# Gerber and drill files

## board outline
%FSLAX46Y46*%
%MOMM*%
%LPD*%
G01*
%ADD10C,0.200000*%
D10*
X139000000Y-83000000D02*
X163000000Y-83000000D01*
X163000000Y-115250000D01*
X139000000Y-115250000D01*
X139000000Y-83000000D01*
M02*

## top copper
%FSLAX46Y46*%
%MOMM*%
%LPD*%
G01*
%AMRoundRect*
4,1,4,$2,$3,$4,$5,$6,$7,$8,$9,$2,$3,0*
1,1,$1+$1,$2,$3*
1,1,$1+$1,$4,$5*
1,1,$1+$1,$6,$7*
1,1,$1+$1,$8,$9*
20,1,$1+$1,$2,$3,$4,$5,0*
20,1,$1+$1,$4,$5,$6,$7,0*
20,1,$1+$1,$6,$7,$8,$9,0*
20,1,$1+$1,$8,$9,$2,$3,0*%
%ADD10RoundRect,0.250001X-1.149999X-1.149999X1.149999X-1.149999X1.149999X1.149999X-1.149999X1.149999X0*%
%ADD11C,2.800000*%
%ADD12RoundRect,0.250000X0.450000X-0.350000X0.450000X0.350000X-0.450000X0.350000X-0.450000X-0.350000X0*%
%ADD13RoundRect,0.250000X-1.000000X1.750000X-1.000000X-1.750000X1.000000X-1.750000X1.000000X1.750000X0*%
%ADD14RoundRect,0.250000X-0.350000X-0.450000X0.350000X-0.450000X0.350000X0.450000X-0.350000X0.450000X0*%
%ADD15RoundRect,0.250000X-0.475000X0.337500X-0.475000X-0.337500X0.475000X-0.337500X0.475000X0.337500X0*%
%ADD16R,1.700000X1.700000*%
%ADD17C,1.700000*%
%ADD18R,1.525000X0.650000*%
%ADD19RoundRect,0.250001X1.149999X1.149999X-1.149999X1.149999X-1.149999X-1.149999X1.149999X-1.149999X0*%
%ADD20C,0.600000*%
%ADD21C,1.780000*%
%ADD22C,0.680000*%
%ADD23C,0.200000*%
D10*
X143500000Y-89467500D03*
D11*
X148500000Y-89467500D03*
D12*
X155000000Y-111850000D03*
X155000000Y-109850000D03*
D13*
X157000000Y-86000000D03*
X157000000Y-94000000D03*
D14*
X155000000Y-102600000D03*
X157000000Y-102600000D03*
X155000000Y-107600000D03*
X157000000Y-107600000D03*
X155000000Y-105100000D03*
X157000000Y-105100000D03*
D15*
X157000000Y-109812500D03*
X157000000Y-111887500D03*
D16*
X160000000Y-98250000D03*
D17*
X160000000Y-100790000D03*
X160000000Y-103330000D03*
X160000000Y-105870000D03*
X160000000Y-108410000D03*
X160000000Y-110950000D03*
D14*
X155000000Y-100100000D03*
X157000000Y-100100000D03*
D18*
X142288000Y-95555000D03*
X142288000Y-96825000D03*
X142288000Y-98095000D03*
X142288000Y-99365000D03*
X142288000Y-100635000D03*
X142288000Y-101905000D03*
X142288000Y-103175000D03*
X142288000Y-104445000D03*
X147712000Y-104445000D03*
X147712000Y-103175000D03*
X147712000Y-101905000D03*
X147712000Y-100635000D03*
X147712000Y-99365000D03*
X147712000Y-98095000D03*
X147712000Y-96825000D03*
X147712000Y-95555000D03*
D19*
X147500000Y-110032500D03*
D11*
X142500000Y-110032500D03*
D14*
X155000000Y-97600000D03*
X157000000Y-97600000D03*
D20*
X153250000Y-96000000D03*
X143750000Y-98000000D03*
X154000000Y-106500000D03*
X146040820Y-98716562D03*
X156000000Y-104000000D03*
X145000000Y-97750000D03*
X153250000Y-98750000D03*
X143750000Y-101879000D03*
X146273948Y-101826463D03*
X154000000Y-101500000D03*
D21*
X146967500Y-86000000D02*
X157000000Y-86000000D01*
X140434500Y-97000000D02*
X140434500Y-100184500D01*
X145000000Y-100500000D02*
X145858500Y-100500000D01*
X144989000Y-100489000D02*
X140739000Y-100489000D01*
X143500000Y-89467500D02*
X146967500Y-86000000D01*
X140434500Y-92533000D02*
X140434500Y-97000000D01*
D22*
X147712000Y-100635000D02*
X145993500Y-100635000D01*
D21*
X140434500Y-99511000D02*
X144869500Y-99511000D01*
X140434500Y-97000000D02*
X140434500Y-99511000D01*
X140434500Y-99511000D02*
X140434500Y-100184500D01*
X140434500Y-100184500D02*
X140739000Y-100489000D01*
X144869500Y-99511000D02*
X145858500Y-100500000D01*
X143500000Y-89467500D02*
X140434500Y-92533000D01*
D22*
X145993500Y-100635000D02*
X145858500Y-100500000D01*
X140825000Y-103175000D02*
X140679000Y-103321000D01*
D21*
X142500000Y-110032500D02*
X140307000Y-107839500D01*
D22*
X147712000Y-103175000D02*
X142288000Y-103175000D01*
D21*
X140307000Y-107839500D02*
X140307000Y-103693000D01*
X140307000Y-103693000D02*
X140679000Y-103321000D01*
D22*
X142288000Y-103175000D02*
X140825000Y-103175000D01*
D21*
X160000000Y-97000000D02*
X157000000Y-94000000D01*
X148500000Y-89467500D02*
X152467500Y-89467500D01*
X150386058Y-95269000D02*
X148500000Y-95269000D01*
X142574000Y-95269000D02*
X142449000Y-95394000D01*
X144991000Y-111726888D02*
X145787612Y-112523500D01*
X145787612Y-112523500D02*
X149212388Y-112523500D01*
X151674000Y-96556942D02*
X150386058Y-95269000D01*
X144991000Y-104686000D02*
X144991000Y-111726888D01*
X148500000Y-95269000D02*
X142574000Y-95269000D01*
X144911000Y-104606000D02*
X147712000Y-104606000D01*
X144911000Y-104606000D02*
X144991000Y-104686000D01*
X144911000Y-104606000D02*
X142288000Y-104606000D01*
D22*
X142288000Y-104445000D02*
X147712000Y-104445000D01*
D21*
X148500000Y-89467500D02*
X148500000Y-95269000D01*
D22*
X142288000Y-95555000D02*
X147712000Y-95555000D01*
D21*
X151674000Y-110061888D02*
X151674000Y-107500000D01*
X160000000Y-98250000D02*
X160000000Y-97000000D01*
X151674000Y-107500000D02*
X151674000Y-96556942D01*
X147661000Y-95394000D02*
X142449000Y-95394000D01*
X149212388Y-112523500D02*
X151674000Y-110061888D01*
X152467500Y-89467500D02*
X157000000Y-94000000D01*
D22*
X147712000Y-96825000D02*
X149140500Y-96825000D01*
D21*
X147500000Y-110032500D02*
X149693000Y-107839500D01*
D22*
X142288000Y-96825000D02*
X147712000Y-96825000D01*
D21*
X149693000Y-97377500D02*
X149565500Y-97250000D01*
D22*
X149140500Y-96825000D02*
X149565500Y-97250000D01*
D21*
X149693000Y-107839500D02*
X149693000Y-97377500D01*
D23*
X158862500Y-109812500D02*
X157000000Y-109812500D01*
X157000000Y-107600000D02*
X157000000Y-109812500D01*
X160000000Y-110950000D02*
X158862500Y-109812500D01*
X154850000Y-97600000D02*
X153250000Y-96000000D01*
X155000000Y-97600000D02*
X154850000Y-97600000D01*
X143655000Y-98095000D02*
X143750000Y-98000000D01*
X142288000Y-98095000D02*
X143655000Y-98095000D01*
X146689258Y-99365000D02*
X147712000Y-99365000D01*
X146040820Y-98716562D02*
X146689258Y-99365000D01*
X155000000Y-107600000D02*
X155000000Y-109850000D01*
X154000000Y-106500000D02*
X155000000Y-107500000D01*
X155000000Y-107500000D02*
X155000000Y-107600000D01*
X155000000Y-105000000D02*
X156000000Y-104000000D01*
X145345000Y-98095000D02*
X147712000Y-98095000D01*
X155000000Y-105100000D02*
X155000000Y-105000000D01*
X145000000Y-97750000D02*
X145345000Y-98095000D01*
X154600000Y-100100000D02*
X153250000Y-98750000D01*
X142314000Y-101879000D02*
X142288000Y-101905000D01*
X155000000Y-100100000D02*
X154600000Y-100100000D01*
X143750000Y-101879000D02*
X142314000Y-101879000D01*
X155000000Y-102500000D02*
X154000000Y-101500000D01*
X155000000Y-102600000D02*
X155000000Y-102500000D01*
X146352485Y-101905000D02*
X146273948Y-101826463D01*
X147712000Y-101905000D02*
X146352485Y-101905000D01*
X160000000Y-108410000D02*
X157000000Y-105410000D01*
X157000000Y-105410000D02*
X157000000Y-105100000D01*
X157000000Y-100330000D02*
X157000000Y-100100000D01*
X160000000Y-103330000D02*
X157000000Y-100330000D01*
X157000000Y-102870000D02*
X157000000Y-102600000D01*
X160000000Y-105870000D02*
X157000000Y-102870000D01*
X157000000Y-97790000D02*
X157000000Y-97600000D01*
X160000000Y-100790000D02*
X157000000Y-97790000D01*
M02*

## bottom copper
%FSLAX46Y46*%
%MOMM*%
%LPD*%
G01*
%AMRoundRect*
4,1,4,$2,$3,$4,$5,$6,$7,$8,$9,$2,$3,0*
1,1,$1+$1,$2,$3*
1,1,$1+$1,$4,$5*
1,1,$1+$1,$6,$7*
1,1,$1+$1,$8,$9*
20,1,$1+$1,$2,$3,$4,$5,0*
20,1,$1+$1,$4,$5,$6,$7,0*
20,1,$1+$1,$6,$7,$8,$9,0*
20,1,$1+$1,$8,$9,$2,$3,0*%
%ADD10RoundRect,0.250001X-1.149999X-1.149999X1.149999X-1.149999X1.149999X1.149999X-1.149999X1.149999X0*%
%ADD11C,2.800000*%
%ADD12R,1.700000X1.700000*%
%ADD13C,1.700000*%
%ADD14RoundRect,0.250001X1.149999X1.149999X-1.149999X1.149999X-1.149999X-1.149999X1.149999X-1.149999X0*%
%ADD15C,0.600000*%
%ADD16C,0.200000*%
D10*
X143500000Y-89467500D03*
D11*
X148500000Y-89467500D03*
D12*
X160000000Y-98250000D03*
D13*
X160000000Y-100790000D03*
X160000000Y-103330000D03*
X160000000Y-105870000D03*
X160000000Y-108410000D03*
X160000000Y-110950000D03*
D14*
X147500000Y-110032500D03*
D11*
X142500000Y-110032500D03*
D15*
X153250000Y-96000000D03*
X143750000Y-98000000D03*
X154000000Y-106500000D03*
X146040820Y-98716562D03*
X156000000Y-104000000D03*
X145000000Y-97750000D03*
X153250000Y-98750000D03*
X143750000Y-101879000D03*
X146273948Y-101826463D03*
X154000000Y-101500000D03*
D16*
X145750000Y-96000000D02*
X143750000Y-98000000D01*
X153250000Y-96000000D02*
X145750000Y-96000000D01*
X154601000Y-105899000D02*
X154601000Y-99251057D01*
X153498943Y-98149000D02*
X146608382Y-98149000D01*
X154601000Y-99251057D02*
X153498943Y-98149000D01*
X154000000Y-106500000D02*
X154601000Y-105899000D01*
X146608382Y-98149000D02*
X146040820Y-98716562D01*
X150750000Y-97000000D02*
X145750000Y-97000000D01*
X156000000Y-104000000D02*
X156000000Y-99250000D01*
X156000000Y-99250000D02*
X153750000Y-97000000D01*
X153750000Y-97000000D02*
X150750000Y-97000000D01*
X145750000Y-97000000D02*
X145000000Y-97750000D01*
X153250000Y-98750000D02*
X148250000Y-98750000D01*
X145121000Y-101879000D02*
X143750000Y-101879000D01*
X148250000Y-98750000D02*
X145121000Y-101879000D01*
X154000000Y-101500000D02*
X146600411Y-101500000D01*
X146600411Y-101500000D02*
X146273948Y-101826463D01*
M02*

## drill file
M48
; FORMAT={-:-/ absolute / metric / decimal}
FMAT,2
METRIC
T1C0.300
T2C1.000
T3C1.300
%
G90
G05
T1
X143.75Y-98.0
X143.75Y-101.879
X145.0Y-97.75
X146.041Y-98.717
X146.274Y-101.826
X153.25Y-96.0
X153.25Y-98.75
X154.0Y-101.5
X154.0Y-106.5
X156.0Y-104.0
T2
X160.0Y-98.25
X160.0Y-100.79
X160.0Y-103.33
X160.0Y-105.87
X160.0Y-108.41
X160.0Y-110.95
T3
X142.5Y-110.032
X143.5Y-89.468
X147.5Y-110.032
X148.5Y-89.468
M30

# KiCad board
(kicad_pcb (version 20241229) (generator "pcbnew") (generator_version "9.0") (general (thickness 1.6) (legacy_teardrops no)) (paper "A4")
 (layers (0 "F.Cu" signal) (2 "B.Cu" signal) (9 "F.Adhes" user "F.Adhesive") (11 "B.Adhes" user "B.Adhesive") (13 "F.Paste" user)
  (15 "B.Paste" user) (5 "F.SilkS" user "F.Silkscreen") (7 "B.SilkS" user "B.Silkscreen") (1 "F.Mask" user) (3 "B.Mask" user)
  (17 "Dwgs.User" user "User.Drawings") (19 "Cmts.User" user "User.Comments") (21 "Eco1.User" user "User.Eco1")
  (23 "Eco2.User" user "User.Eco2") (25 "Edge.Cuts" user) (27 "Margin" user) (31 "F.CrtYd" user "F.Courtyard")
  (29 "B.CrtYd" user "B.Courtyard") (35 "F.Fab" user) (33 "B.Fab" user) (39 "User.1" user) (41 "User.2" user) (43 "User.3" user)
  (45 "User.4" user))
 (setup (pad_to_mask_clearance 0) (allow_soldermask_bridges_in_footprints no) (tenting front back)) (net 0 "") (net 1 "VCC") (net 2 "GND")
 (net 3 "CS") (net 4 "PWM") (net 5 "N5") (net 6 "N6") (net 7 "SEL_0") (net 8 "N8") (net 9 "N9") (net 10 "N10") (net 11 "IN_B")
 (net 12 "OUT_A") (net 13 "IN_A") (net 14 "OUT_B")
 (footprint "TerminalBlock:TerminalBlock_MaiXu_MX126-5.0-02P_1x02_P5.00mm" (layer "F.Cu") (at 143.5 89.4675)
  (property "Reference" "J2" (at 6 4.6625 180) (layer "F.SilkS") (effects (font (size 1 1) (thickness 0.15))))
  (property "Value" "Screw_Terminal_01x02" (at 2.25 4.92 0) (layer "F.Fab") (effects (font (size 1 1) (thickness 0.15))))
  (pad "1" thru_hole roundrect (at 0 0) (size 2.8 2.8) (drill 1.3) (layers "*.Cu" "*.Mask") (remove_unused_layers no)
   (roundrect_rratio 0.089286) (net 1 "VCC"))
  (pad "2" thru_hole circle (at 5 0) (size 2.8 2.8) (drill 1.3) (layers "*.Cu" "*.Mask") (remove_unused_layers no) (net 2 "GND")))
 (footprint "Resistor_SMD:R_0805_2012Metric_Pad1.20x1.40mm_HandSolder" (layer "F.Cu") (at 155 110.85 90)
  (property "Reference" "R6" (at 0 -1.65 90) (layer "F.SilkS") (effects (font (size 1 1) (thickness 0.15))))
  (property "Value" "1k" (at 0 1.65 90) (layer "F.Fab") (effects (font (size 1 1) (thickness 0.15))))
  (pad "1" smd roundrect (at -1 0 90) (size 1.2 1.4) (layers "F.Cu" "F.Mask" "F.Paste") (roundrect_rratio 0.208333) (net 2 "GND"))
  (pad "2" smd roundrect (at 1 0 90) (size 1.2 1.4) (layers "F.Cu" "F.Mask" "F.Paste") (roundrect_rratio 0.208333) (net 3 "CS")))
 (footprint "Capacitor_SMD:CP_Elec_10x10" (layer "F.Cu") (at 157 90 -90)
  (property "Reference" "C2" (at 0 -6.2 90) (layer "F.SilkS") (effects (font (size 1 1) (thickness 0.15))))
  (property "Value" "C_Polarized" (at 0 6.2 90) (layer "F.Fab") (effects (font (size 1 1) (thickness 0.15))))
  (pad "1" smd roundrect (at -4 0 270) (size 4 2.5) (layers "F.Cu" "F.Mask" "F.Paste") (roundrect_rratio 0.1) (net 1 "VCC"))
  (pad "2" smd roundrect (at 4 0 270) (size 4 2.5) (layers "F.Cu" "F.Mask" "F.Paste") (roundrect_rratio 0.1) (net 2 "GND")))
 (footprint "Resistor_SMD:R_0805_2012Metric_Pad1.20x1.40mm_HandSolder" (layer "F.Cu") (at 156 102.6)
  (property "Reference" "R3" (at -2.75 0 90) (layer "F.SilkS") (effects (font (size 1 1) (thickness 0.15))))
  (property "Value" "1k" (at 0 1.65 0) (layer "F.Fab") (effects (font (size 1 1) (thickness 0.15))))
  (pad "1" smd roundrect (at -1 0) (size 1.2 1.4) (layers "F.Cu" "F.Mask" "F.Paste") (roundrect_rratio 0.208333) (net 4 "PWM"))
  (pad "2" smd roundrect (at 1 0) (size 1.2 1.4) (layers "F.Cu" "F.Mask" "F.Paste") (roundrect_rratio 0.208333) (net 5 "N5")))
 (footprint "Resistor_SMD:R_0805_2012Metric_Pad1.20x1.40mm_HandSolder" (layer "F.Cu") (at 156 107.6)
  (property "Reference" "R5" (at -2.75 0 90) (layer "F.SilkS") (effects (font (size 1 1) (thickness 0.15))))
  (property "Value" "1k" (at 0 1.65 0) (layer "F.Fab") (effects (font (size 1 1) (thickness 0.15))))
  (pad "1" smd roundrect (at -1 0) (size 1.2 1.4) (layers "F.Cu" "F.Mask" "F.Paste") (roundrect_rratio 0.208333) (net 3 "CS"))
  (pad "2" smd roundrect (at 1 0) (size 1.2 1.4) (layers "F.Cu" "F.Mask" "F.Paste") (roundrect_rratio 0.208333) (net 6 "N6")))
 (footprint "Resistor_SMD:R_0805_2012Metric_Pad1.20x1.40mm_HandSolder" (layer "F.Cu") (at 156 105.1)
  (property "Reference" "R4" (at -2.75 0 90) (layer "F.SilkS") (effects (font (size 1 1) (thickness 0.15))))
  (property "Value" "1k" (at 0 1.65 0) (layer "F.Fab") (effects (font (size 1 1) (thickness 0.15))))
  (pad "1" smd roundrect (at -1 0) (size 1.2 1.4) (layers "F.Cu" "F.Mask" "F.Paste") (roundrect_rratio 0.208333) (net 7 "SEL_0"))
  (pad "2" smd roundrect (at 1 0) (size 1.2 1.4) (layers "F.Cu" "F.Mask" "F.Paste") (roundrect_rratio 0.208333) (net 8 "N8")))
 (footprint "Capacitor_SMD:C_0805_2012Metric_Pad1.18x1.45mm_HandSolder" (layer "F.Cu") (at 157 110.85 -90)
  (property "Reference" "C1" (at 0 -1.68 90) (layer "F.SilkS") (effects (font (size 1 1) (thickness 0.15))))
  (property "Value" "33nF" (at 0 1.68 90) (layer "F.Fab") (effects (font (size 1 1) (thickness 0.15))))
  (pad "1" smd roundrect (at -1.0375 0 270) (size 1.175 1.45) (layers "F.Cu" "F.Mask" "F.Paste") (roundrect_rratio 0.212766) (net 6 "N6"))
  (pad "2" smd roundrect (at 1.0375 0 270) (size 1.175 1.45) (layers "F.Cu" "F.Mask" "F.Paste") (roundrect_rratio 0.212766) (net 2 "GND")))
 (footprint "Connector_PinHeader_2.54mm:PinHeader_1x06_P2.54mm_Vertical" (layer "F.Cu") (at 160 98.25)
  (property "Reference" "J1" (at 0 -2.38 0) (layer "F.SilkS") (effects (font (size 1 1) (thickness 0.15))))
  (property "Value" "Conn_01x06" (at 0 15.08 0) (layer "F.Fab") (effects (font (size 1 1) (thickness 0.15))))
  (pad "1" thru_hole rect (at 0 0) (size 1.7 1.7) (drill 1) (layers "*.Cu" "*.Mask") (remove_unused_layers no) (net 2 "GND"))
  (pad "2" thru_hole circle (at 0 2.54) (size 1.7 1.7) (drill 1) (layers "*.Cu" "*.Mask") (remove_unused_layers no) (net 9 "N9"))
  (pad "3" thru_hole circle (at 0 5.08) (size 1.7 1.7) (drill 1) (layers "*.Cu" "*.Mask") (remove_unused_layers no) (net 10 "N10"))
  (pad "4" thru_hole circle (at 0 7.62) (size 1.7 1.7) (drill 1) (layers "*.Cu" "*.Mask") (remove_unused_layers no) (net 5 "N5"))
  (pad "5" thru_hole circle (at 0 10.16) (size 1.7 1.7) (drill 1) (layers "*.Cu" "*.Mask") (remove_unused_layers no) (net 8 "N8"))
  (pad "6" thru_hole circle (at 0 12.7) (size 1.7 1.7) (drill 1) (layers "*.Cu" "*.Mask") (remove_unused_layers no) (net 6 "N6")))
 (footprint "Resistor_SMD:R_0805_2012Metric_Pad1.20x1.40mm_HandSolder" (layer "F.Cu") (at 156 100.1)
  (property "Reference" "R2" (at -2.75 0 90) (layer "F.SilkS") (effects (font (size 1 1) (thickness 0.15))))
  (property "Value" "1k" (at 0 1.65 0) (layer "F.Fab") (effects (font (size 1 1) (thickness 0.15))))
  (pad "1" smd roundrect (at -1 0) (size 1.2 1.4) (layers "F.Cu" "F.Mask" "F.Paste") (roundrect_rratio 0.208333) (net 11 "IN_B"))
  (pad "2" smd roundrect (at 1 0) (size 1.2 1.4) (layers "F.Cu" "F.Mask" "F.Paste") (roundrect_rratio 0.208333) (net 10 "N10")))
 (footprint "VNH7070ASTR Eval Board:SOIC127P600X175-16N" (layer "F.Cu") (at 145 100)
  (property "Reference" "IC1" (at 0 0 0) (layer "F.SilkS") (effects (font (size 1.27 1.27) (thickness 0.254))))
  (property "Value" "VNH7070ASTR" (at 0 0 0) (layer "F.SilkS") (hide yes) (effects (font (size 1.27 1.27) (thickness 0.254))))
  (pad "1" smd rect (at -2.712 -4.445 90) (size 0.65 1.525) (layers "F.Cu" "F.Mask" "F.Paste") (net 2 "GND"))
  (pad "2" smd rect (at -2.712 -3.175 90) (size 0.65 1.525) (layers "F.Cu" "F.Mask" "F.Paste") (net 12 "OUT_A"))
  (pad "3" smd rect (at -2.712 -1.905 90) (size 0.65 1.525) (layers "F.Cu" "F.Mask" "F.Paste") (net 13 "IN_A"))
  (pad "4" smd rect (at -2.712 -0.635 90) (size 0.65 1.525) (layers "F.Cu" "F.Mask" "F.Paste") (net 1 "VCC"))
  (pad "5" smd rect (at -2.712 0.635 90) (size 0.65 1.525) (layers "F.Cu" "F.Mask" "F.Paste") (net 1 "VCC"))
  (pad "6" smd rect (at -2.712 1.905 90) (size 0.65 1.525) (layers "F.Cu" "F.Mask" "F.Paste") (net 11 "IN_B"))
  (pad "7" smd rect (at -2.712 3.175 90) (size 0.65 1.525) (layers "F.Cu" "F.Mask" "F.Paste") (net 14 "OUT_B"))
  (pad "8" smd rect (at -2.712 4.445 90) (size 0.65 1.525) (layers "F.Cu" "F.Mask" "F.Paste") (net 2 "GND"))
  (pad "9" smd rect (at 2.712 4.445 90) (size 0.65 1.525) (layers "F.Cu" "F.Mask" "F.Paste") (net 2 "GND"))
  (pad "10" smd rect (at 2.712 3.175 90) (size 0.65 1.525) (layers "F.Cu" "F.Mask" "F.Paste") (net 14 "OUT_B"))
  (pad "11" smd rect (at 2.712 1.905 90) (size 0.65 1.525) (layers "F.Cu" "F.Mask" "F.Paste") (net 4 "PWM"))
  (pad "12" smd rect (at 2.712 0.635 90) (size 0.65 1.525) (layers "F.Cu" "F.Mask" "F.Paste") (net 1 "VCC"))
  (pad "13" smd rect (at 2.712 -0.635 90) (size 0.65 1.525) (layers "F.Cu" "F.Mask" "F.Paste") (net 3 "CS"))
  (pad "14" smd rect (at 2.712 -1.905 90) (size 0.65 1.525) (layers "F.Cu" "F.Mask" "F.Paste") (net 7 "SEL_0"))
  (pad "15" smd rect (at 2.712 -3.175 90) (size 0.65 1.525) (layers "F.Cu" "F.Mask" "F.Paste") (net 12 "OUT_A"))
  (pad "16" smd rect (at 2.712 -4.445 90) (size 0.65 1.525) (layers "F.Cu" "F.Mask" "F.Paste") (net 2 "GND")))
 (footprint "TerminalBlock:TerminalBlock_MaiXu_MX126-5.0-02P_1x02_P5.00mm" (layer "F.Cu") (at 147.5 110.0325 180)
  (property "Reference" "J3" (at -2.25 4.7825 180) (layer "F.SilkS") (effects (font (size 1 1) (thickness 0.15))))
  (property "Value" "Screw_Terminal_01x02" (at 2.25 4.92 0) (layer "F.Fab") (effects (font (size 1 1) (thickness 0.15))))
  (pad "1" thru_hole roundrect (at 0 0 180) (size 2.8 2.8) (drill 1.3) (layers "*.Cu" "*.Mask") (remove_unused_layers no)
   (roundrect_rratio 0.089286) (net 12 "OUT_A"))
  (pad "2" thru_hole circle (at 5 0 180) (size 2.8 2.8) (drill 1.3) (layers "*.Cu" "*.Mask") (remove_unused_layers no) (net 14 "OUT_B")))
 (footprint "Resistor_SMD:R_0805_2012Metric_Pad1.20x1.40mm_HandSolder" (layer "F.Cu") (at 156 97.6)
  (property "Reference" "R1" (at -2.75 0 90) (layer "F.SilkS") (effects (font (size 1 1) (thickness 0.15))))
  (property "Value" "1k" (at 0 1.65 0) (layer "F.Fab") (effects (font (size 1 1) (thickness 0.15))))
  (pad "1" smd roundrect (at -1 0) (size 1.2 1.4) (layers "F.Cu" "F.Mask" "F.Paste") (roundrect_rratio 0.208333) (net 13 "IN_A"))
  (pad "2" smd roundrect (at 1 0) (size 1.2 1.4) (layers "F.Cu" "F.Mask" "F.Paste") (roundrect_rratio 0.208333) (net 9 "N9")))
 (gr_rect (start 139 83) (end 163 115.25) (stroke (width 0.2) (type solid)) (fill no) (layer "Edge.Cuts"))
 (segment (start 146.9675 86) (end 157 86) (width 1.78) (layer "F.Cu") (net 1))
 (segment (start 140.4345 97) (end 140.4345 100.1845) (width 1.78) (layer "F.Cu") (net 1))
 (segment (start 145 100.5) (end 145.8585 100.5) (width 1.78) (layer "F.Cu") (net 1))
 (segment (start 144.989 100.489) (end 140.739 100.489) (width 1.78) (layer "F.Cu") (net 1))
 (segment (start 143.5 89.4675) (end 146.9675 86) (width 1.78) (layer "F.Cu") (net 1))
 (segment (start 140.4345 92.533) (end 140.4345 97) (width 1.78) (layer "F.Cu") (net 1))
 (segment (start 147.712 100.635) (end 145.9935 100.635) (width 0.68) (layer "F.Cu") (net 1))
 (segment (start 140.4345 99.511) (end 144.8695 99.511) (width 1.78) (layer "F.Cu") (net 1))
 (segment (start 140.4345 97) (end 140.4345 99.511) (width 1.78) (layer "F.Cu") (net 1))
 (segment (start 140.4345 99.511) (end 140.4345 100.1845) (width 1.78) (layer "F.Cu") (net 1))
 (segment (start 140.4345 100.1845) (end 140.739 100.489) (width 1.78) (layer "F.Cu") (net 1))
 (segment (start 144.8695 99.511) (end 145.8585 100.5) (width 1.78) (layer "F.Cu") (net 1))
 (segment (start 143.5 89.4675) (end 140.4345 92.533) (width 1.78) (layer "F.Cu") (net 1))
 (segment (start 145.9935 100.635) (end 145.8585 100.5) (width 0.68) (layer "F.Cu") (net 1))
 (segment (start 140.825 103.175) (end 140.679 103.321) (width 0.68) (layer "F.Cu") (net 14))
 (segment (start 142.5 110.0325) (end 140.307 107.8395) (width 1.78) (layer "F.Cu") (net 14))
 (segment (start 147.712 103.175) (end 142.288 103.175) (width 0.68) (layer "F.Cu") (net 14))
 (segment (start 140.307 107.8395) (end 140.307 103.693) (width 1.78) (layer "F.Cu") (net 14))
 (segment (start 140.307 103.693) (end 140.679 103.321) (width 1.78) (layer "F.Cu") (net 14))
 (segment (start 142.288 103.175) (end 140.825 103.175) (width 0.68) (layer "F.Cu") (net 14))
 (segment (start 160 97) (end 157 94) (width 1.78) (layer "F.Cu") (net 2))
 (segment (start 148.5 89.4675) (end 152.4675 89.4675) (width 1.78) (layer "F.Cu") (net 2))
 (segment (start 150.386058 95.269) (end 148.5 95.269) (width 1.78) (layer "F.Cu") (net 2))
 (segment (start 142.574 95.269) (end 142.449 95.394) (width 1.78) (layer "F.Cu") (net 2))
 (segment (start 144.991 111.726888) (end 145.787612 112.5235) (width 1.78) (layer "F.Cu") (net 2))
 (segment (start 145.787612 112.5235) (end 149.212388 112.5235) (width 1.78) (layer "F.Cu") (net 2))
 (segment (start 151.674 96.556942) (end 150.386058 95.269) (width 1.78) (layer "F.Cu") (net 2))
 (segment (start 144.991 104.686) (end 144.991 111.726888) (width 1.78) (layer "F.Cu") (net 2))
 (segment (start 148.5 95.269) (end 142.574 95.269) (width 1.78) (layer "F.Cu") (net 2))
 (segment (start 144.911 104.606) (end 147.712 104.606) (width 1.78) (layer "F.Cu") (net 2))
 (segment (start 144.911 104.606) (end 144.991 104.686) (width 1.78) (layer "F.Cu") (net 2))
 (segment (start 144.911 104.606) (end 142.288 104.606) (width 1.78) (layer "F.Cu") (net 2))
 (segment (start 142.288 104.445) (end 147.712 104.445) (width 0.68) (layer "F.Cu") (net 2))
 (segment (start 148.5 89.4675) (end 148.5 95.269) (width 1.78) (layer "F.Cu") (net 2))
 (segment (start 142.288 95.555) (end 147.712 95.555) (width 0.68) (layer "F.Cu") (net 2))
 (segment (start 151.674 110.061888) (end 151.674 107.5) (width 1.78) (layer "F.Cu") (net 2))
 (segment (start 160 98.25) (end 160 97) (width 1.78) (layer "F.Cu") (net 2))
 (segment (start 151.674 107.5) (end 151.674 96.556942) (width 1.78) (layer "F.Cu") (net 2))
 (segment (start 147.661 95.394) (end 142.449 95.394) (width 1.78) (layer "F.Cu") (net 2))
 (segment (start 149.212388 112.5235) (end 151.674 110.061888) (width 1.78) (layer "F.Cu") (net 2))
 (segment (start 152.4675 89.4675) (end 157 94) (width 1.78) (layer "F.Cu") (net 2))
 (segment (start 147.712 96.825) (end 149.1405 96.825) (width 0.68) (layer "F.Cu") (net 12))
 (segment (start 147.5 110.0325) (end 149.693 107.8395) (width 1.78) (layer "F.Cu") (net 12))
 (segment (start 142.288 96.825) (end 147.712 96.825) (width 0.68) (layer "F.Cu") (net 12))
 (segment (start 149.693 97.3775) (end 149.5655 97.25) (width 1.78) (layer "F.Cu") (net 12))
 (segment (start 149.1405 96.825) (end 149.5655 97.25) (width 0.68) (layer "F.Cu") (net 12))
 (segment (start 149.693 107.8395) (end 149.693 97.3775) (width 1.78) (layer "F.Cu") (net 12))
 (segment (start 158.8625 109.8125) (end 157 109.8125) (width 0.2) (layer "F.Cu") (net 6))
 (segment (start 157 107.6) (end 157 109.8125) (width 0.2) (layer "F.Cu") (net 6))
 (segment (start 160 110.95) (end 158.8625 109.8125) (width 0.2) (layer "F.Cu") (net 6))
 (segment (start 154.85 97.6) (end 153.25 96) (width 0.2) (layer "F.Cu") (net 13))
 (segment (start 155 97.6) (end 154.85 97.6) (width 0.2) (layer "F.Cu") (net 13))
 (segment (start 143.655 98.095) (end 143.75 98) (width 0.2) (layer "F.Cu") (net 13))
 (segment (start 142.288 98.095) (end 143.655 98.095) (width 0.2) (layer "F.Cu") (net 13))
 (via (at 153.25 96) (size 0.6) (drill 0.3) (layers "F.Cu" "B.Cu") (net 13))
 (via (at 143.75 98) (size 0.6) (drill 0.3) (layers "F.Cu" "B.Cu") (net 13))
 (segment (start 145.75 96) (end 143.75 98) (width 0.2) (layer "B.Cu") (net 13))
 (segment (start 153.25 96) (end 145.75 96) (width 0.2) (layer "B.Cu") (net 13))
 (segment (start 146.689258 99.365) (end 147.712 99.365) (width 0.2) (layer "F.Cu") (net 3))
 (segment (start 146.04082 98.716562) (end 146.689258 99.365) (width 0.2) (layer "F.Cu") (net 3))
 (segment (start 155 107.6) (end 155 109.85) (width 0.2) (layer "F.Cu") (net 3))
 (segment (start 154 106.5) (end 155 107.5) (width 0.2) (layer "F.Cu") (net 3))
 (segment (start 155 107.5) (end 155 107.6) (width 0.2) (layer "F.Cu") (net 3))
 (via (at 154 106.5) (size 0.6) (drill 0.3) (layers "F.Cu" "B.Cu") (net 3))
 (via (at 146.04082 98.716562) (size 0.6) (drill 0.3) (layers "F.Cu" "B.Cu") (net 3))
 (segment (start 154.601 105.899) (end 154.601 99.251057) (width 0.2) (layer "B.Cu") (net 3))
 (segment (start 153.498943 98.149) (end 146.608382 98.149) (width 0.2) (layer "B.Cu") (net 3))
 (segment (start 154.601 99.251057) (end 153.498943 98.149) (width 0.2) (layer "B.Cu") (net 3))
 (segment (start 154 106.5) (end 154.601 105.899) (width 0.2) (layer "B.Cu") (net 3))
 (segment (start 146.608382 98.149) (end 146.04082 98.716562) (width 0.2) (layer "B.Cu") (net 3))
 (segment (start 155 105) (end 156 104) (width 0.2) (layer "F.Cu") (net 7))
 (segment (start 145.345 98.095) (end 147.712 98.095) (width 0.2) (layer "F.Cu") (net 7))
 (segment (start 155 105.1) (end 155 105) (width 0.2) (layer "F.Cu") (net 7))
 (segment (start 145 97.75) (end 145.345 98.095) (width 0.2) (layer "F.Cu") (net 7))
 (via (at 156 104) (size 0.6) (drill 0.3) (layers "F.Cu" "B.Cu") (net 7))
 (via (at 145 97.75) (size 0.6) (drill 0.3) (layers "F.Cu" "B.Cu") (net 7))
 (segment (start 150.75 97) (end 145.75 97) (width 0.2) (layer "B.Cu") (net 7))
 (segment (start 156 104) (end 156 99.25) (width 0.2) (layer "B.Cu") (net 7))
 (segment (start 156 99.25) (end 153.75 97) (width 0.2) (layer "B.Cu") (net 7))
 (segment (start 153.75 97) (end 150.75 97) (width 0.2) (layer "B.Cu") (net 7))
 (segment (start 145.75 97) (end 145 97.75) (width 0.2) (layer "B.Cu") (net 7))
 (segment (start 154.6 100.1) (end 153.25 98.75) (width 0.2) (layer "F.Cu") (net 11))
 (segment (start 142.314 101.879) (end 142.288 101.905) (width 0.2) (layer "F.Cu") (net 11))
 (segment (start 155 100.1) (end 154.6 100.1) (width 0.2) (layer "F.Cu") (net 11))
 (segment (start 143.75 101.879) (end 142.314 101.879) (width 0.2) (layer "F.Cu") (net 11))
 (via (at 153.25 98.75) (size 0.6) (drill 0.3) (layers "F.Cu" "B.Cu") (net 11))
 (via (at 143.75 101.879) (size 0.6) (drill 0.3) (layers "F.Cu" "B.Cu") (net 11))
 (segment (start 153.25 98.75) (end 148.25 98.75) (width 0.2) (layer "B.Cu") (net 11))
 (segment (start 145.121 101.879) (end 143.75 101.879) (width 0.2) (layer "B.Cu") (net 11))
 (segment (start 148.25 98.75) (end 145.121 101.879) (width 0.2) (layer "B.Cu") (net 11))
 (segment (start 155 102.5) (end 154 101.5) (width 0.2) (layer "F.Cu") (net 4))
 (segment (start 155 102.6) (end 155 102.5) (width 0.2) (layer "F.Cu") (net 4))
 (segment (start 146.352485 101.905) (end 146.273948 101.826463) (width 0.2) (layer "F.Cu") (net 4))
 (segment (start 147.712 101.905) (end 146.352485 101.905) (width 0.2) (layer "F.Cu") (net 4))
 (via (at 146.273948 101.826463) (size 0.6) (drill 0.3) (layers "F.Cu" "B.Cu") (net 4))
 (via (at 154 101.5) (size 0.6) (drill 0.3) (layers "F.Cu" "B.Cu") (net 4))
 (segment (start 154 101.5) (end 146.600411 101.5) (width 0.2) (layer "B.Cu") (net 4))
 (segment (start 146.600411 101.5) (end 146.273948 101.826463) (width 0.2) (layer "B.Cu") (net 4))
 (segment (start 160 108.41) (end 157 105.41) (width 0.2) (layer "F.Cu") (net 8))
 (segment (start 157 105.41) (end 157 105.1) (width 0.2) (layer "F.Cu") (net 8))
 (segment (start 157 100.33) (end 157 100.1) (width 0.2) (layer "F.Cu") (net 10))
 (segment (start 160 103.33) (end 157 100.33) (width 0.2) (layer "F.Cu") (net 10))
 (segment (start 157 102.87) (end 157 102.6) (width 0.2) (layer "F.Cu") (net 5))
 (segment (start 160 105.87) (end 157 102.87) (width 0.2) (layer "F.Cu") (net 5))
 (segment (start 157 97.79) (end 157 97.6) (width 0.2) (layer "F.Cu") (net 9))
 (segment (start 160 100.79) (end 157 97.79) (width 0.2) (layer "F.Cu") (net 9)))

